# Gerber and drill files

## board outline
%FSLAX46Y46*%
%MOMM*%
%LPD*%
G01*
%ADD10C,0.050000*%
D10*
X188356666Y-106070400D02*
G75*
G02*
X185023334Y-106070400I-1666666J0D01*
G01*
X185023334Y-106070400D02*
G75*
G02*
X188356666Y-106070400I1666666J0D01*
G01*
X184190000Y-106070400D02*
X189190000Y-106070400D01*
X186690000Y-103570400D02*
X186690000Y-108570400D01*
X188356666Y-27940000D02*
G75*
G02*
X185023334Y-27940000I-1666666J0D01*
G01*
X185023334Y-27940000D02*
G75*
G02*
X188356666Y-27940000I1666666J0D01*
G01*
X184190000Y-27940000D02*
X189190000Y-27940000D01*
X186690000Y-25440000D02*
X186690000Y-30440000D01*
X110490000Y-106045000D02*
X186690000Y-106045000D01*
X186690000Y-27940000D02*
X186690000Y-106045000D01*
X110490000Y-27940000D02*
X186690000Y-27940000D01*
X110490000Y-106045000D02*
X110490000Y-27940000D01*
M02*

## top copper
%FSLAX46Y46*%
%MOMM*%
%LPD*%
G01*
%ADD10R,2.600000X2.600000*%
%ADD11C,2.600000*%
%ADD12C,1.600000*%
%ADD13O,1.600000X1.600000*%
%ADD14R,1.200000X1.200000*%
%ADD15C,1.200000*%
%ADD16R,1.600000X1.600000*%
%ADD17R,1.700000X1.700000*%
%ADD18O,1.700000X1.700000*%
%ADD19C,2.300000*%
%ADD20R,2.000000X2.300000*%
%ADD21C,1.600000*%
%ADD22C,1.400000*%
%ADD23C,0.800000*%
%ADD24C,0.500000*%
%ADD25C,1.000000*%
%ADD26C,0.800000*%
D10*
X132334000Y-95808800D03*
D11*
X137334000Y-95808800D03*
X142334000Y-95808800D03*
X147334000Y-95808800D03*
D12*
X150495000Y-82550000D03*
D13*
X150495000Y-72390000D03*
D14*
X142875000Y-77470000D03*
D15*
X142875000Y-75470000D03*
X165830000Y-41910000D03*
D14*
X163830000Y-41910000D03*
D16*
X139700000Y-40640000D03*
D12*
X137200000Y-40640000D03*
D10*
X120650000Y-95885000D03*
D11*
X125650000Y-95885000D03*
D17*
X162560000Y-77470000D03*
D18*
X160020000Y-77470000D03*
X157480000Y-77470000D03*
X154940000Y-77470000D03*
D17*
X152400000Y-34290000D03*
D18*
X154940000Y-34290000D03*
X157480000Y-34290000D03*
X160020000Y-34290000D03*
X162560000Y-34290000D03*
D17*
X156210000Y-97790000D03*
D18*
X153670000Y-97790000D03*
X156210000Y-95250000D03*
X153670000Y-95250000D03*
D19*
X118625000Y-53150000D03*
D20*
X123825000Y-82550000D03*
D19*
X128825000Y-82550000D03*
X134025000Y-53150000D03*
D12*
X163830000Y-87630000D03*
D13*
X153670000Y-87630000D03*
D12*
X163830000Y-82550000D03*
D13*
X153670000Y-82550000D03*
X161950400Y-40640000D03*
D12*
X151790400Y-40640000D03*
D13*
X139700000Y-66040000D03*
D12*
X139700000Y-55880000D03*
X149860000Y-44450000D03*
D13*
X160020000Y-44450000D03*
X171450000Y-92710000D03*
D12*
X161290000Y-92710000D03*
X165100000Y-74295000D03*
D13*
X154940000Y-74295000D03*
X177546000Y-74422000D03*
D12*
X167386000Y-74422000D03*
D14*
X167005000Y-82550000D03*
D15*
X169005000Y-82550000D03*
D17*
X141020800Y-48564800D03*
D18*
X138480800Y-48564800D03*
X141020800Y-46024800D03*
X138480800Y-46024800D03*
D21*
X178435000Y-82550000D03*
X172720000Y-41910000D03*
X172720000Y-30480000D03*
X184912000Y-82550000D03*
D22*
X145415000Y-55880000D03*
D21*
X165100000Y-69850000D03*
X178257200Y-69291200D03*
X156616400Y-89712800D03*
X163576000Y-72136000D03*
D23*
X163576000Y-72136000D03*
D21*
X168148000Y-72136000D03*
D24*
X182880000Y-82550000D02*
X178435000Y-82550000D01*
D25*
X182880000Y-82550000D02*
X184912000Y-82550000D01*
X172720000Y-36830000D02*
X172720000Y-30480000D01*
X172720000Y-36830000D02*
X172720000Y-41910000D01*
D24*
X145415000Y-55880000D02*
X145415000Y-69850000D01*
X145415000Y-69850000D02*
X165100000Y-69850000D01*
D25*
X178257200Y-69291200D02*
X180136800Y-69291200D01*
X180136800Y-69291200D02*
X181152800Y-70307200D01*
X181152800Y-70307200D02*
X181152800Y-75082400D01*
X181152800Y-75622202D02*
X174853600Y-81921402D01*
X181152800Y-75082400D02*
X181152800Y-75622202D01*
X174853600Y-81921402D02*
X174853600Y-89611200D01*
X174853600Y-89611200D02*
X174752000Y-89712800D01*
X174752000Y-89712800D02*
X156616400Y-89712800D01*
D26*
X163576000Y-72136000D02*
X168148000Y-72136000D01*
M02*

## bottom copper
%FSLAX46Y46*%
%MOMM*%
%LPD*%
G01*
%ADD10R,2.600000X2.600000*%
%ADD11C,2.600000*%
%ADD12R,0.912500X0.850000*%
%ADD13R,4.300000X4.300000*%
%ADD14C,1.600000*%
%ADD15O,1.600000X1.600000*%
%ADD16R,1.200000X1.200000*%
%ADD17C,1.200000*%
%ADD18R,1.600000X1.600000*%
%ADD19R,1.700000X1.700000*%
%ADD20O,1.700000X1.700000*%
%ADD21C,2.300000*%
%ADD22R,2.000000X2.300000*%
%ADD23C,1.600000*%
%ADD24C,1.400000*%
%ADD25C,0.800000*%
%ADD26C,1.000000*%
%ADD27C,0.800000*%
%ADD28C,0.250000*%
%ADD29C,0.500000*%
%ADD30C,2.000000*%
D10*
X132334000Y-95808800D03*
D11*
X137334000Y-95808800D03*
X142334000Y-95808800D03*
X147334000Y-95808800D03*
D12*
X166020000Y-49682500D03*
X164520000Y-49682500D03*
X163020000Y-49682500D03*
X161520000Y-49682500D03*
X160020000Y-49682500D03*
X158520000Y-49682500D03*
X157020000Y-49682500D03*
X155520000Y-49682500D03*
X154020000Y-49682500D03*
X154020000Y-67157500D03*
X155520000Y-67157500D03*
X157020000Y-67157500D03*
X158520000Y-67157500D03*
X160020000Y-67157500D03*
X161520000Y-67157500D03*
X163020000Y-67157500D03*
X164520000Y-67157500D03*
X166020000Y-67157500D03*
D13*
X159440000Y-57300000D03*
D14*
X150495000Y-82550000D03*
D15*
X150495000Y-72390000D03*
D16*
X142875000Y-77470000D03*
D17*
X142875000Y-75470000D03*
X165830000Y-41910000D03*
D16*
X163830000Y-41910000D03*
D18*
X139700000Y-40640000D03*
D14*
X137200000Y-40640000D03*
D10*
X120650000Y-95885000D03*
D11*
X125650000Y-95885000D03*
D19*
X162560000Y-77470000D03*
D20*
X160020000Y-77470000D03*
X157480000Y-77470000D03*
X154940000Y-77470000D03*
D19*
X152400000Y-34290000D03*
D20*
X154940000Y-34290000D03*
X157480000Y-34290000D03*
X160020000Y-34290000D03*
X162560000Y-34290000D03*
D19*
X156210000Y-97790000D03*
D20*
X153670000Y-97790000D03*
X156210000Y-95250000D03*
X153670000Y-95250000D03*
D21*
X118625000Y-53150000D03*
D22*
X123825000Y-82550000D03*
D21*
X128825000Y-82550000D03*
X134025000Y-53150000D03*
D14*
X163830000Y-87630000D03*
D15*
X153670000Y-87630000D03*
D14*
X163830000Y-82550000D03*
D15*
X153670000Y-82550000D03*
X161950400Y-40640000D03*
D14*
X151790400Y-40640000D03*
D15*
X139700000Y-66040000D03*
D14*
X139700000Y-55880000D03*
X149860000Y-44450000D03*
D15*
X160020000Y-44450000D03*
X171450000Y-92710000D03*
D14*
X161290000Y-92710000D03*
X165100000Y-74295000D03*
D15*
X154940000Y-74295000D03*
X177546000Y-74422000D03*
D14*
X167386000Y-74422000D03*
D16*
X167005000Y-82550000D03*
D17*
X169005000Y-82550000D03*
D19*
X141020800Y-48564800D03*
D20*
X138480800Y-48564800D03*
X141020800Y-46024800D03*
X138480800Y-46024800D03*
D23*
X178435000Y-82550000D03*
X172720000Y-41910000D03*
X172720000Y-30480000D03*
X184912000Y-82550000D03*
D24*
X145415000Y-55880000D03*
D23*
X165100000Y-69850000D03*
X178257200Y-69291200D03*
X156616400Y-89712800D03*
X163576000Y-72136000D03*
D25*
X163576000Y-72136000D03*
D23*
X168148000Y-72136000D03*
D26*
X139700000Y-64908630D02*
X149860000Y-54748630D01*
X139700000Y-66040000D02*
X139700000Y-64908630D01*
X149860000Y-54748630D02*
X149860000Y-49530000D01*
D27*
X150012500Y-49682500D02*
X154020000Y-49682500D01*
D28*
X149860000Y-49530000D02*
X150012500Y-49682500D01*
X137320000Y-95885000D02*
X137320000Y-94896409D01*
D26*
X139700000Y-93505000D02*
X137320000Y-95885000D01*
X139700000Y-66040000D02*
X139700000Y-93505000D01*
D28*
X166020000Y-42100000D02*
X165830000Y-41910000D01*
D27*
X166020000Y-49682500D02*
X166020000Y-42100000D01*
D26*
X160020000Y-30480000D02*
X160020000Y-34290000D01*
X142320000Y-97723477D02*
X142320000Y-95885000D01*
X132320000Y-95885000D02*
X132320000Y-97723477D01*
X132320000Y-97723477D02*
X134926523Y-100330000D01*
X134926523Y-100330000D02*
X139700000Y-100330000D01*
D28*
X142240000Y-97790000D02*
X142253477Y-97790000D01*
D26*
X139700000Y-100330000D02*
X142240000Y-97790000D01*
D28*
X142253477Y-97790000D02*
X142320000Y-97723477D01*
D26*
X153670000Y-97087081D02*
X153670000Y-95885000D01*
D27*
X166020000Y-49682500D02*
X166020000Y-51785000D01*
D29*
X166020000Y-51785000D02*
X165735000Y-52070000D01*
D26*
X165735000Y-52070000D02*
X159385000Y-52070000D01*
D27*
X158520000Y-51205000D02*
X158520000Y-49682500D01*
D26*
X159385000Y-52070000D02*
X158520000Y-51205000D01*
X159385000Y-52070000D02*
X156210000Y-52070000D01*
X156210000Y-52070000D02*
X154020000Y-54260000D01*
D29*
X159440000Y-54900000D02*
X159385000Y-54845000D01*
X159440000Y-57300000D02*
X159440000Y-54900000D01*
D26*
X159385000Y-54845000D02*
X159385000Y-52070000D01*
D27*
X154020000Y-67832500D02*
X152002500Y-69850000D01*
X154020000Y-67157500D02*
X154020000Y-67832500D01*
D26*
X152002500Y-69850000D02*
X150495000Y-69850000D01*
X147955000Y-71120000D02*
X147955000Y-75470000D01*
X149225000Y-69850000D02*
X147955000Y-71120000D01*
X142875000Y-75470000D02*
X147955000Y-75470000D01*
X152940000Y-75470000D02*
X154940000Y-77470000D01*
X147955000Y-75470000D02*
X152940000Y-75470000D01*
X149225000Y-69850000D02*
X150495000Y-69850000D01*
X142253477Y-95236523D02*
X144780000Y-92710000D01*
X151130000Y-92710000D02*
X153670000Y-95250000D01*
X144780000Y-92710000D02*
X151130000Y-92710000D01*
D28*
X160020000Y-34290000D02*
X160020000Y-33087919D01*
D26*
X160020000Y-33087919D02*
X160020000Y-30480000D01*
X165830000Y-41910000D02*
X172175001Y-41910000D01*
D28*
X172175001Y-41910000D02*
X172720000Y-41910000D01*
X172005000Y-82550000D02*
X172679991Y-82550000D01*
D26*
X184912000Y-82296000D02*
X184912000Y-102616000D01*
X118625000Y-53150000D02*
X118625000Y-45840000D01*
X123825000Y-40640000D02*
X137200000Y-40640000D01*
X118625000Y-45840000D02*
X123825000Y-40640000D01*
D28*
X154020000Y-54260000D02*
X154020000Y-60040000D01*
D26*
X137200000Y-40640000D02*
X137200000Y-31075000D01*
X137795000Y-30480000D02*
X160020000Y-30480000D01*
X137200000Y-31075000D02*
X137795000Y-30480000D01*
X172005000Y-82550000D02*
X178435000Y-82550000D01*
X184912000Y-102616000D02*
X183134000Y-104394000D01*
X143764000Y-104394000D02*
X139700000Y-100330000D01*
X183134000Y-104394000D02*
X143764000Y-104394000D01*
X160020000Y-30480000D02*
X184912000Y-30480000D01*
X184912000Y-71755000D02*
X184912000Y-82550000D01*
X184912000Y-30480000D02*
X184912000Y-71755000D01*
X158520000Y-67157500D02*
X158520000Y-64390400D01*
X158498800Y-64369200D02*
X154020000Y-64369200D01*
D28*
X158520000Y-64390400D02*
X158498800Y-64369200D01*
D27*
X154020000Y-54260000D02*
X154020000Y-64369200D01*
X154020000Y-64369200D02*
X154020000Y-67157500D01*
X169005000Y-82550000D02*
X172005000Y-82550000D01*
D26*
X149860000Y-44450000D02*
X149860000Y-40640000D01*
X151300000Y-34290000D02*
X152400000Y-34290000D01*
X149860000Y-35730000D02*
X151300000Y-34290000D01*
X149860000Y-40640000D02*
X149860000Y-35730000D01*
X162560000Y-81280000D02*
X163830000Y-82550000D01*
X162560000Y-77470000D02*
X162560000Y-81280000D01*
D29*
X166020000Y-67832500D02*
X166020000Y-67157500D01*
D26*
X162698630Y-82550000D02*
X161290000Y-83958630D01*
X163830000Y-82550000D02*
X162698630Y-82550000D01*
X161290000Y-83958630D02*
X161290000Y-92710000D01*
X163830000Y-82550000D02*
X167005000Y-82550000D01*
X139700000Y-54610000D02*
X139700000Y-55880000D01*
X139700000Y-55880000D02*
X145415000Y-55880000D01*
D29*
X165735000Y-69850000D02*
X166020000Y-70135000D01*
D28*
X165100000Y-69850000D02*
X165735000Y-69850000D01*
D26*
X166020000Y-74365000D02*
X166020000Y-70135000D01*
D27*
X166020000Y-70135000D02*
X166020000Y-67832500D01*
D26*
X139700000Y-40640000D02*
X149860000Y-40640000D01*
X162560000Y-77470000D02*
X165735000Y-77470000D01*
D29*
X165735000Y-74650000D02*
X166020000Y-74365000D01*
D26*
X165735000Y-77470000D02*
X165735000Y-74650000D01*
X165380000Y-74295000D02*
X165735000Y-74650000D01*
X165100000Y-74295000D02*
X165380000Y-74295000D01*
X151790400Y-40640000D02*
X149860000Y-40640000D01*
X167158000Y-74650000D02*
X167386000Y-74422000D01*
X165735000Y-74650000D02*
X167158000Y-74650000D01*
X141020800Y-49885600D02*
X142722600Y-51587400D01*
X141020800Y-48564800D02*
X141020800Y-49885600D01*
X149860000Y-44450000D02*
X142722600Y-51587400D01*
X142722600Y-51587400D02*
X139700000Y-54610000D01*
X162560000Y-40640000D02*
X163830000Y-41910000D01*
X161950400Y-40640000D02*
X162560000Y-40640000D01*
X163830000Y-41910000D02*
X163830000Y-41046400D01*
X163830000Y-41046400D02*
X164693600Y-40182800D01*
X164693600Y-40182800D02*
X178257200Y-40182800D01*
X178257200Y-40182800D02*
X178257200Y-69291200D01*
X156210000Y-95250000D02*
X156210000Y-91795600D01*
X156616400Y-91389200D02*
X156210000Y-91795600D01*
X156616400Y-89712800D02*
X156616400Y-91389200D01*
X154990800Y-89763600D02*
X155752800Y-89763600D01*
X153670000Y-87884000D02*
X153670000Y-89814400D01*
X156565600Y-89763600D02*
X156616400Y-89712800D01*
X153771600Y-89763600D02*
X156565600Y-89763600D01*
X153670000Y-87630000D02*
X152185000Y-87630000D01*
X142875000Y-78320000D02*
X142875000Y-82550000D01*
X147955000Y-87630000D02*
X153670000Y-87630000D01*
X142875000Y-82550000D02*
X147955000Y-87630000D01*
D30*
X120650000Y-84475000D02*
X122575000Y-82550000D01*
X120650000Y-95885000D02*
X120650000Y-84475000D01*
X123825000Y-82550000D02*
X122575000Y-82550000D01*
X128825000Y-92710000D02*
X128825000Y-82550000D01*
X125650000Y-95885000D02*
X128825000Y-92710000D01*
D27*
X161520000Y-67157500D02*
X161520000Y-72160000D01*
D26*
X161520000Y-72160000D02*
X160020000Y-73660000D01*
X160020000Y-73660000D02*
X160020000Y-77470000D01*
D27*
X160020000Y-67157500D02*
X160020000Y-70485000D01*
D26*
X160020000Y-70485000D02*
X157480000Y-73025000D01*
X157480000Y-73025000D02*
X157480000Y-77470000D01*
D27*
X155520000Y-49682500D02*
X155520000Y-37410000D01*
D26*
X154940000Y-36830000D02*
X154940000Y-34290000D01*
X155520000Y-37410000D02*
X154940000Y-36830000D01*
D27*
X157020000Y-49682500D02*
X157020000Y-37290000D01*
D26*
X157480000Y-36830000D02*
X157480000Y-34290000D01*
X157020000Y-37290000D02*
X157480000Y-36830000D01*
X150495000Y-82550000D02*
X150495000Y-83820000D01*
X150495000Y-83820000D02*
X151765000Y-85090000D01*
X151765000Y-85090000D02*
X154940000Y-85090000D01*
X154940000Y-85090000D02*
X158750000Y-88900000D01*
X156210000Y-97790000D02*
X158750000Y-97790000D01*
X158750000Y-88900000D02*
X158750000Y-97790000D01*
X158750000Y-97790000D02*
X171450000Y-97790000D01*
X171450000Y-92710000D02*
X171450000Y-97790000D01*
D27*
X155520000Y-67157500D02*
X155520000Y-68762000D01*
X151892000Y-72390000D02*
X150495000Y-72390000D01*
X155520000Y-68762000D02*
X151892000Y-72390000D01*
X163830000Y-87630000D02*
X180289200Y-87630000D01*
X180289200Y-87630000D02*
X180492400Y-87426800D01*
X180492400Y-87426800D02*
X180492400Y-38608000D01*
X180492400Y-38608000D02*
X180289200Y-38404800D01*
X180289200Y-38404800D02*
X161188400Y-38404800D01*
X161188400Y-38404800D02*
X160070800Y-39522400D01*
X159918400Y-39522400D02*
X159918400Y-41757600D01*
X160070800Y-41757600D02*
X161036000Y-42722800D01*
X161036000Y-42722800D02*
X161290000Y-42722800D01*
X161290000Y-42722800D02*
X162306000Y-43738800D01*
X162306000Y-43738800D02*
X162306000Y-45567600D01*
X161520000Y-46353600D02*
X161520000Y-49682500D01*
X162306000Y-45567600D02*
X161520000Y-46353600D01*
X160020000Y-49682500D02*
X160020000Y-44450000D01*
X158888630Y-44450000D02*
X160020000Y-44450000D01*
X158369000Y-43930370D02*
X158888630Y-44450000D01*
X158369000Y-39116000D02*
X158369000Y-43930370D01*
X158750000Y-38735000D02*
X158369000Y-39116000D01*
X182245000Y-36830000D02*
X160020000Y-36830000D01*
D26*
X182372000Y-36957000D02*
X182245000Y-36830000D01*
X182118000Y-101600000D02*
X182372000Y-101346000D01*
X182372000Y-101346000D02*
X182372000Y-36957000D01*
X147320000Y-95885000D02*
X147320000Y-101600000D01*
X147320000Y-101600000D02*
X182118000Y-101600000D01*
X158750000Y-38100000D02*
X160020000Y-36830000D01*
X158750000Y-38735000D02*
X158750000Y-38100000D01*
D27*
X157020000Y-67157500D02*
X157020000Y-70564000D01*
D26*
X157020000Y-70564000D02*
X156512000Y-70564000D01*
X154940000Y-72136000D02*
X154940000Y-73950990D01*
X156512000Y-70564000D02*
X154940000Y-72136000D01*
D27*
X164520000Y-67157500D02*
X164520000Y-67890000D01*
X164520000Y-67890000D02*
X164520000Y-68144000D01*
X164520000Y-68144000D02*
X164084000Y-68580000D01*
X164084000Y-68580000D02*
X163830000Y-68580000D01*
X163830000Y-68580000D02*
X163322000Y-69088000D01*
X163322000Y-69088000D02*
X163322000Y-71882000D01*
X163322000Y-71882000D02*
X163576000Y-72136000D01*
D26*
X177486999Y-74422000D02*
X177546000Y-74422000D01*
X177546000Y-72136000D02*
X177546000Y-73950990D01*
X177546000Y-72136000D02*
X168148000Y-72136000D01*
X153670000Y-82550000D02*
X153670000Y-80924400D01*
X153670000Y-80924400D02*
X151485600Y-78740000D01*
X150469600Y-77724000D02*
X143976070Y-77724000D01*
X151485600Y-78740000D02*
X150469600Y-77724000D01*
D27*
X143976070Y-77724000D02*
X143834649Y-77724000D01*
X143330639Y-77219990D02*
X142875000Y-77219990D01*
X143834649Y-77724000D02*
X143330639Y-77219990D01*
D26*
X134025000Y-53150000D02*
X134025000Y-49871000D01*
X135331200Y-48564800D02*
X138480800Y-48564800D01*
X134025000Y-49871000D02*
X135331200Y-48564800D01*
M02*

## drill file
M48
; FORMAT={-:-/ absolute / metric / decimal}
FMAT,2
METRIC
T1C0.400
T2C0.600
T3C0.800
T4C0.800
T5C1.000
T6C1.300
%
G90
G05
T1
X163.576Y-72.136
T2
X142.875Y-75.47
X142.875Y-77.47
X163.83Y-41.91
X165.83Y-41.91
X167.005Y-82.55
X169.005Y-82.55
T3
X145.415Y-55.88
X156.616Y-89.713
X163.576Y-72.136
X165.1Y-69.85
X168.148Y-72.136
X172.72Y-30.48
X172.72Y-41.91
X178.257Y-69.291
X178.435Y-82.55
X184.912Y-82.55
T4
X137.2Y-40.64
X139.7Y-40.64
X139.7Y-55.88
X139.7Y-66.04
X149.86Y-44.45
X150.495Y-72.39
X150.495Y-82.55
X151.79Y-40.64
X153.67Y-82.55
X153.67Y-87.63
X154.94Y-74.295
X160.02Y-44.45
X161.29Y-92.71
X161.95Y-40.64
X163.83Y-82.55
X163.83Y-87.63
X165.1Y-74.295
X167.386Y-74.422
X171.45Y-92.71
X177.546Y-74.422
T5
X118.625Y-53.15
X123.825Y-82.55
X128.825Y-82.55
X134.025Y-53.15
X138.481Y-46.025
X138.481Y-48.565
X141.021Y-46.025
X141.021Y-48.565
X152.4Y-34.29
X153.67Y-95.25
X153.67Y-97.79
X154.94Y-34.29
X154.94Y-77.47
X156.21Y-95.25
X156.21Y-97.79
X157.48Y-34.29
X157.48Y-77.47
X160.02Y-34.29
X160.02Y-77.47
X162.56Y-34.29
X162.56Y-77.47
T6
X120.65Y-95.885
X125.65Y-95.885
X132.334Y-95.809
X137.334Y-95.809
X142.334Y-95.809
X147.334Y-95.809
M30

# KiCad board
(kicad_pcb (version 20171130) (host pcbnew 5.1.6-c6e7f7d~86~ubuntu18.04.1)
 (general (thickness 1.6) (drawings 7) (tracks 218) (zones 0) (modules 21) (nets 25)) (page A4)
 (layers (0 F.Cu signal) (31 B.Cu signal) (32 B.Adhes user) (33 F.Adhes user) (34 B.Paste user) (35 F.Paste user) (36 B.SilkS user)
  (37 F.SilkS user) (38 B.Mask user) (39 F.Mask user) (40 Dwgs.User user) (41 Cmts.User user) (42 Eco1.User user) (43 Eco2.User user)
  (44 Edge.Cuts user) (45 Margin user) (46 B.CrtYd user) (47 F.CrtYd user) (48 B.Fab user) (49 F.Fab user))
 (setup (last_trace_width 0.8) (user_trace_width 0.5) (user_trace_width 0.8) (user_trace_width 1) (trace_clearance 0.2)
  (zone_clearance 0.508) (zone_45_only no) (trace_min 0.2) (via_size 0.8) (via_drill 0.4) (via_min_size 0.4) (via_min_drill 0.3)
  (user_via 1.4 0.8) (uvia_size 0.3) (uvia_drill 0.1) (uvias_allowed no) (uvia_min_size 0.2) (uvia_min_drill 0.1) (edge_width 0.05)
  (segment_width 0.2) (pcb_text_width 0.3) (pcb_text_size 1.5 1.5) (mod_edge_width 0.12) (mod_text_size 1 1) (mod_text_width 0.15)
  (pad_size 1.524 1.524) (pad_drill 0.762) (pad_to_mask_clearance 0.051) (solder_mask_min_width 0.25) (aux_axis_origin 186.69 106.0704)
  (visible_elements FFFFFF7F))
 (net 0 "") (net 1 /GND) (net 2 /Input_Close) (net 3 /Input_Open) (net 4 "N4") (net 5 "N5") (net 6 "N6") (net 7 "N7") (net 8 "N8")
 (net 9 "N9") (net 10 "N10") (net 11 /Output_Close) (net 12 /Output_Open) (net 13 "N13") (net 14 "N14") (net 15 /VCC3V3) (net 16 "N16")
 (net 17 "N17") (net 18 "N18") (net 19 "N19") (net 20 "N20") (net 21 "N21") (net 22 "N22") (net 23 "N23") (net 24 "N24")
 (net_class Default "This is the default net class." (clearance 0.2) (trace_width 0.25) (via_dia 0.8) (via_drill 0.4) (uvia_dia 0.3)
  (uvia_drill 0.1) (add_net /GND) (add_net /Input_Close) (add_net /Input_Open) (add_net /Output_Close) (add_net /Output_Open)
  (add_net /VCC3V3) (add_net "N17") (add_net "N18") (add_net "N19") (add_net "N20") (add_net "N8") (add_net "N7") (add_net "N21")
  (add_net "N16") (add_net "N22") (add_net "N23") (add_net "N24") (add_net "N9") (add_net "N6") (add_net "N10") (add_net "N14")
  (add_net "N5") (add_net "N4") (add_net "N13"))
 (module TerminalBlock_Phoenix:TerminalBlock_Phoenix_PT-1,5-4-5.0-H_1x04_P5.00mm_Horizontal (layer F.Cu) (at 132.334 95.8088)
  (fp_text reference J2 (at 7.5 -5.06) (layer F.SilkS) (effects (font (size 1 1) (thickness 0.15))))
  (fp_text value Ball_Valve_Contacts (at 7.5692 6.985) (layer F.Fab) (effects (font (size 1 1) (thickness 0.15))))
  (pad 4 thru_hole rect (at 0 0) (size 2.6 2.6) (drill 1.3) (layers *.Cu *.Mask) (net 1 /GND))
  (pad 3 thru_hole circle (at 5 0) (size 2.6 2.6) (drill 1.3) (layers *.Cu *.Mask) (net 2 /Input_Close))
  (pad 2 thru_hole circle (at 10 0) (size 2.6 2.6) (drill 1.3) (layers *.Cu *.Mask) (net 1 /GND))
  (pad 1 thru_hole circle (at 15 0) (size 2.6 2.6) (drill 1.3) (layers *.Cu *.Mask) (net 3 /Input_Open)))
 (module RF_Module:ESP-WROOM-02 (layer B.Cu) (at 160.02 58.42 90)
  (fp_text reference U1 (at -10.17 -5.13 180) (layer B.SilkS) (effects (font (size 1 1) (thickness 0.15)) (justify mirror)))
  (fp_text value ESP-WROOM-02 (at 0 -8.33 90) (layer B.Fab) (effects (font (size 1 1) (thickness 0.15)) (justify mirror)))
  (pad 18 smd rect (at 8.7375 6 90) (size 0.85 0.9125) (layers B.Cu B.Paste B.Mask) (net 1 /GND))
  (pad 17 smd rect (at 8.7375 4.5 90) (size 0.85 0.9125) (layers B.Cu B.Paste B.Mask) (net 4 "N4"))
  (pad 16 smd rect (at 8.7375 3 90) (size 0.85 0.9125) (layers B.Cu B.Paste B.Mask) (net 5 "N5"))
  (pad 15 smd rect (at 8.7375 1.5 90) (size 0.85 0.9125) (layers B.Cu B.Paste B.Mask) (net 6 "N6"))
  (pad 14 smd rect (at 8.7375 0 90) (size 0.85 0.9125) (layers B.Cu B.Paste B.Mask) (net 3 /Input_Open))
  (pad 13 smd rect (at 8.7375 -1.5 90) (size 0.85 0.9125) (layers B.Cu B.Paste B.Mask) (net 1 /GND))
  (pad 12 smd rect (at 8.7375 -3 90) (size 0.85 0.9125) (layers B.Cu B.Paste B.Mask) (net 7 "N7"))
  (pad 11 smd rect (at 8.7375 -4.5 90) (size 0.85 0.9125) (layers B.Cu B.Paste B.Mask) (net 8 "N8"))
  (pad 10 smd rect (at 8.7375 -6 90) (size 0.85 0.9125) (layers B.Cu B.Paste B.Mask) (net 2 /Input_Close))
  (pad 9 smd rect (at -8.7375 -6 90) (size 0.85 0.9125) (layers B.Cu B.Paste B.Mask) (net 1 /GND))
  (pad 8 smd rect (at -8.7375 -4.5 90) (size 0.85 0.9125) (layers B.Cu B.Paste B.Mask) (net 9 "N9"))
  (pad 7 smd rect (at -8.7375 -3 90) (size 0.85 0.9125) (layers B.Cu B.Paste B.Mask) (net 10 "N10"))
  (pad 6 smd rect (at -8.7375 -1.5 90) (size 0.85 0.9125) (layers B.Cu B.Paste B.Mask) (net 1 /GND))
  (pad 5 smd rect (at -8.7375 0 90) (size 0.85 0.9125) (layers B.Cu B.Paste B.Mask) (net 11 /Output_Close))
  (pad 4 smd rect (at -8.7375 1.5 90) (size 0.85 0.9125) (layers B.Cu B.Paste B.Mask) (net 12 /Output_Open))
  (pad 3 smd rect (at -8.7375 3 90) (size 0.85 0.9125) (layers B.Cu B.Paste B.Mask) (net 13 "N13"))
  (pad 2 smd rect (at -8.7375 4.5 90) (size 0.85 0.9125) (layers B.Cu B.Paste B.Mask) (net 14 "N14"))
  (pad 1 smd rect (at -8.7375 6 90) (size 0.85 0.9125) (layers B.Cu B.Paste B.Mask) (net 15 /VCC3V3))
  (pad 19 smd rect (at 1.12 -0.58 90) (size 4.3 4.3) (layers B.Cu B.Paste B.Mask) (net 1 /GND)))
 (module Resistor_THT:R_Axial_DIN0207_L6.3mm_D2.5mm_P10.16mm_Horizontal (layer F.Cu) (at 150.495 82.55 90)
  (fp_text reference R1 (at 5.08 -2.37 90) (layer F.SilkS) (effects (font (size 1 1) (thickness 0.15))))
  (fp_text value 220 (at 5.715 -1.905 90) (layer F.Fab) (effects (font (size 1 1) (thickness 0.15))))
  (pad 1 thru_hole circle (at 0 0 90) (size 1.6 1.6) (drill 0.8) (layers *.Cu *.Mask) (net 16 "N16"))
  (pad 2 thru_hole oval (at 10.16 0 90) (size 1.6 1.6) (drill 0.8) (layers *.Cu *.Mask) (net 9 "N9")))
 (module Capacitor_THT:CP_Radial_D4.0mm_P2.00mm (layer F.Cu) (at 142.875 77.47 90)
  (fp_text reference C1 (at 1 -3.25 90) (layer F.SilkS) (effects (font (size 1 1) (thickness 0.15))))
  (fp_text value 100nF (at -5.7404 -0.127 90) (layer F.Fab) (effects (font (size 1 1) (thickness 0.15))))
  (pad 1 thru_hole rect (at 0 0 90) (size 1.2 1.2) (drill 0.6) (layers *.Cu *.Mask) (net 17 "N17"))
  (pad 2 thru_hole circle (at 2 0 90) (size 1.2 1.2) (drill 0.6) (layers *.Cu *.Mask) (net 1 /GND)))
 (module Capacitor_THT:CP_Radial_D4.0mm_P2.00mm (layer F.Cu) (at 163.83 41.91)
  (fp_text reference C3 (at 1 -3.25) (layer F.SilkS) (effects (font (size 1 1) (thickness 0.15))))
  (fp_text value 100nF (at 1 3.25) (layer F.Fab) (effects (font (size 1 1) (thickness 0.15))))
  (pad 2 thru_hole circle (at 2 0) (size 1.2 1.2) (drill 0.6) (layers *.Cu *.Mask) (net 1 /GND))
  (pad 1 thru_hole rect (at 0 0) (size 1.2 1.2) (drill 0.6) (layers *.Cu *.Mask) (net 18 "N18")))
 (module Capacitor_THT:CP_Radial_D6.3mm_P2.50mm (layer F.Cu) (at 139.7 40.64 180)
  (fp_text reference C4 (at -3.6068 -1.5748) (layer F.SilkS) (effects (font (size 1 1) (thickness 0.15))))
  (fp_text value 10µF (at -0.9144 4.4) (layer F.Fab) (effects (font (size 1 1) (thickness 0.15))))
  (pad 1 thru_hole rect (at 0 0 180) (size 1.6 1.6) (drill 0.8) (layers *.Cu *.Mask) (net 15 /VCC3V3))
  (pad 2 thru_hole circle (at 2.5 0 180) (size 1.6 1.6) (drill 0.8) (layers *.Cu *.Mask) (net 1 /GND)))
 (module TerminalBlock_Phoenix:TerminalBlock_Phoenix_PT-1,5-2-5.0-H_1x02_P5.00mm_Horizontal (layer F.Cu) (at 120.65 95.885)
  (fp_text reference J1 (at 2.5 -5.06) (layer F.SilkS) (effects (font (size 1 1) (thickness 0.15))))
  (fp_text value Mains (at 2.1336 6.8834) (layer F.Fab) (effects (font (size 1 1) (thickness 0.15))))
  (pad 1 thru_hole rect (at 0 0) (size 2.6 2.6) (drill 1.3) (layers *.Cu *.Mask) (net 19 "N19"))
  (pad 2 thru_hole circle (at 5 0) (size 2.6 2.6) (drill 1.3) (layers *.Cu *.Mask) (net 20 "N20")))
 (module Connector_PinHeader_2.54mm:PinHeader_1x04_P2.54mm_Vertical (layer F.Cu) (at 162.56 77.47 270)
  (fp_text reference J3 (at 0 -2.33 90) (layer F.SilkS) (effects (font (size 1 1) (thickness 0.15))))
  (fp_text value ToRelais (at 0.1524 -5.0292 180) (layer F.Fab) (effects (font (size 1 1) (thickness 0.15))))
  (pad 1 thru_hole rect (at 0 0 270) (size 1.7 1.7) (drill 1) (layers *.Cu *.Mask) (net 15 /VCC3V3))
  (pad 2 thru_hole oval (at 0 2.54 270) (size 1.7 1.7) (drill 1) (layers *.Cu *.Mask) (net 12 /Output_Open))
  (pad 3 thru_hole oval (at 0 5.08 270) (size 1.7 1.7) (drill 1) (layers *.Cu *.Mask) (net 11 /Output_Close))
  (pad 4 thru_hole oval (at 0 7.62 270) (size 1.7 1.7) (drill 1) (layers *.Cu *.Mask) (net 1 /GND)))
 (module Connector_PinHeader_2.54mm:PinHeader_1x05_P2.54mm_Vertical (layer F.Cu) (at 152.4 34.29 90)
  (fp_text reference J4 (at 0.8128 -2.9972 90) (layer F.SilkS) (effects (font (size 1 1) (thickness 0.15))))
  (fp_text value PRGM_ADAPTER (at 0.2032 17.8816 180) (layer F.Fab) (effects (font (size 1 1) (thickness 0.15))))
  (pad 1 thru_hole rect (at 0 0 90) (size 1.7 1.7) (drill 1) (layers *.Cu *.Mask) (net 15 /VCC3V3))
  (pad 2 thru_hole oval (at 0 2.54 90) (size 1.7 1.7) (drill 1) (layers *.Cu *.Mask) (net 8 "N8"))
  (pad 3 thru_hole oval (at 0 5.08 90) (size 1.7 1.7) (drill 1) (layers *.Cu *.Mask) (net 7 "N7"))
  (pad 4 thru_hole oval (at 0 7.62 90) (size 1.7 1.7) (drill 1) (layers *.Cu *.Mask) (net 1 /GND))
  (pad 5 thru_hole oval (at 0 10.16 90) (size 1.7 1.7) (drill 1) (layers *.Cu *.Mask) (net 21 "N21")))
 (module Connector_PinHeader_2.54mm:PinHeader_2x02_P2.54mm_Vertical (layer F.Cu) (at 156.21 97.79 180)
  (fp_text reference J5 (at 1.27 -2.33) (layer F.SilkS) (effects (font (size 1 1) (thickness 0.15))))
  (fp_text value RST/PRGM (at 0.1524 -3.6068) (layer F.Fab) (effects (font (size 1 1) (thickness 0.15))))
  (pad 1 thru_hole rect (at 0 0 180) (size 1.7 1.7) (drill 1) (layers *.Cu *.Mask) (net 16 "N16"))
  (pad 2 thru_hole oval (at 2.54 0 180) (size 1.7 1.7) (drill 1) (layers *.Cu *.Mask) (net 1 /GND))
  (pad 3 thru_hole oval (at 0 2.54 180) (size 1.7 1.7) (drill 1) (layers *.Cu *.Mask) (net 18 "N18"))
  (pad 4 thru_hole oval (at 2.54 2.54 180) (size 1.7 1.7) (drill 1) (layers *.Cu *.Mask) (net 1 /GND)))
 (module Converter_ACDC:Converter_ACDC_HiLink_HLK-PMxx (layer F.Cu) (at 123.825 82.55 90)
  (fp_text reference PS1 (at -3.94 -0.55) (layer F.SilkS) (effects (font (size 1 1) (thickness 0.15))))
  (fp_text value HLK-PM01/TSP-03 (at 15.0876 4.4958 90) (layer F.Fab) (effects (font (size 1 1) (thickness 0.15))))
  (pad 3 thru_hole circle (at 29.4 -5.2 90) (size 2.3 2.3) (drill 1) (layers *.Cu *.Mask) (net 1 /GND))
  (pad 1 thru_hole rect (at 0 0 90) (size 2.3 2) (drill 1) (layers *.Cu *.Mask) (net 19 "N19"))
  (pad 2 thru_hole circle (at 0 5 90) (size 2.3 2.3) (drill 1) (layers *.Cu *.Mask) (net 20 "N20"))
  (pad 4 thru_hole circle (at 29.4 10.2 90) (size 2.3 2.3) (drill 1) (layers *.Cu *.Mask) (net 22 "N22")))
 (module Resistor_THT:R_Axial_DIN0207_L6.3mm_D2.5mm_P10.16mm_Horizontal (layer F.Cu) (at 163.83 87.63 180)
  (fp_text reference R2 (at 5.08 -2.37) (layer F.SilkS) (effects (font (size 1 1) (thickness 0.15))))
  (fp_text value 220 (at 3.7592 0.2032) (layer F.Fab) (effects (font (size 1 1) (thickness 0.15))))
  (pad 1 thru_hole circle (at 0 0 180) (size 1.6 1.6) (drill 0.8) (layers *.Cu *.Mask) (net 6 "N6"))
  (pad 2 thru_hole oval (at 10.16 0 180) (size 1.6 1.6) (drill 0.8) (layers *.Cu *.Mask) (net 18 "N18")))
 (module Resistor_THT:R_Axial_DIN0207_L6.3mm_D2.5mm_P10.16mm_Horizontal (layer F.Cu) (at 163.83 82.55 180)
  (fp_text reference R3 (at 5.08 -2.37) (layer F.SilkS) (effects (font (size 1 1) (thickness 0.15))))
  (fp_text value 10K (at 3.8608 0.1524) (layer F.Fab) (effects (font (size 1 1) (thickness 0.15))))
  (pad 1 thru_hole circle (at 0 0 180) (size 1.6 1.6) (drill 0.8) (layers *.Cu *.Mask) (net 15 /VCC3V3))
  (pad 2 thru_hole oval (at 10.16 0 180) (size 1.6 1.6) (drill 0.8) (layers *.Cu *.Mask) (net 17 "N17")))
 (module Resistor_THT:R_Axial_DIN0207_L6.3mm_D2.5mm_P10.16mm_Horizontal (layer F.Cu) (at 151.7904 40.64)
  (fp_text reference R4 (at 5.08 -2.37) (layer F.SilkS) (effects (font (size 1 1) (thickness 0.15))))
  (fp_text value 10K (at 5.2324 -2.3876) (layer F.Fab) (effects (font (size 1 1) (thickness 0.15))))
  (pad 2 thru_hole oval (at 10.16 0) (size 1.6 1.6) (drill 0.8) (layers *.Cu *.Mask) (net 18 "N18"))
  (pad 1 thru_hole circle (at 0 0) (size 1.6 1.6) (drill 0.8) (layers *.Cu *.Mask) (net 15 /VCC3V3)))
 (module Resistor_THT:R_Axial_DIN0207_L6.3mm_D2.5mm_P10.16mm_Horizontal (layer F.Cu) (at 139.7 55.88 270)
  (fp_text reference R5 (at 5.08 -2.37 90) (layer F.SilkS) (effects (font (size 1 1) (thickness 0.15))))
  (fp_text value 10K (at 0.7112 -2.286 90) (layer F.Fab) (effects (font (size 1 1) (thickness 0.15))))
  (pad 2 thru_hole oval (at 10.16 0 270) (size 1.6 1.6) (drill 0.8) (layers *.Cu *.Mask) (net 2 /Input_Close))
  (pad 1 thru_hole circle (at 0 0 270) (size 1.6 1.6) (drill 0.8) (layers *.Cu *.Mask) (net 15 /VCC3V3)))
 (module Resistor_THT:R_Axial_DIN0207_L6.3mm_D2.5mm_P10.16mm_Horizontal (layer F.Cu) (at 149.86 44.45)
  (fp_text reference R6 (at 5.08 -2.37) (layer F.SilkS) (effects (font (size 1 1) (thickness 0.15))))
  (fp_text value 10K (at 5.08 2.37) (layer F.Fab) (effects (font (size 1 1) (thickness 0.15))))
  (pad 1 thru_hole circle (at 0 0) (size 1.6 1.6) (drill 0.8) (layers *.Cu *.Mask) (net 15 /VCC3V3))
  (pad 2 thru_hole oval (at 10.16 0) (size 1.6 1.6) (drill 0.8) (layers *.Cu *.Mask) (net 3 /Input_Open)))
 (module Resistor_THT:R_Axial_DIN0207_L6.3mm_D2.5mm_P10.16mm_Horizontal (layer F.Cu) (at 161.29 92.71)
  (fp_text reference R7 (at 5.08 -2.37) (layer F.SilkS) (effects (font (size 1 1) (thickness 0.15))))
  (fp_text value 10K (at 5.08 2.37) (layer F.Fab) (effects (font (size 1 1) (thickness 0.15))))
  (pad 2 thru_hole oval (at 10.16 0) (size 1.6 1.6) (drill 0.8) (layers *.Cu *.Mask) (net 16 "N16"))
  (pad 1 thru_hole circle (at 0 0) (size 1.6 1.6) (drill 0.8) (layers *.Cu *.Mask) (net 15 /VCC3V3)))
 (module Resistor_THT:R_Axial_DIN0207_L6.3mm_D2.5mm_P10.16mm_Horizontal (layer F.Cu) (at 165.1 74.295 180)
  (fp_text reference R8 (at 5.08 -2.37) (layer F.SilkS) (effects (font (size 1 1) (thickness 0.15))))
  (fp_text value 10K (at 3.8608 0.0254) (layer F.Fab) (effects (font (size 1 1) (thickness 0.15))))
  (pad 1 thru_hole circle (at 0 0 180) (size 1.6 1.6) (drill 0.8) (layers *.Cu *.Mask) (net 15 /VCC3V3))
  (pad 2 thru_hole oval (at 10.16 0 180) (size 1.6 1.6) (drill 0.8) (layers *.Cu *.Mask) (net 10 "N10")))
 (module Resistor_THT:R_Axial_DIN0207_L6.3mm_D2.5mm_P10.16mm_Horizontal (layer F.Cu) (at 167.386 74.422)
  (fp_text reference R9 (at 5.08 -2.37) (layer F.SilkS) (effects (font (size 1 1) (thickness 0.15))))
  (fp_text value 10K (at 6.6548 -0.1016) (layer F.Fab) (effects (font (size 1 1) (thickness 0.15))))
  (pad 2 thru_hole oval (at 10.16 0) (size 1.6 1.6) (drill 0.8) (layers *.Cu *.Mask) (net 14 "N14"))
  (pad 1 thru_hole circle (at 0 0) (size 1.6 1.6) (drill 0.8) (layers *.Cu *.Mask) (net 15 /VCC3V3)))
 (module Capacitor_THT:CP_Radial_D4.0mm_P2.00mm (layer F.Cu) (at 167.005 82.55)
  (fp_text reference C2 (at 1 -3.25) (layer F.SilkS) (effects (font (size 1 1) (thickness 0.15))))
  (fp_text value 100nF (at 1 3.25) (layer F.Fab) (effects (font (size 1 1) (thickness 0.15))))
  (pad 1 thru_hole rect (at 0 0) (size 1.2 1.2) (drill 0.6) (layers *.Cu *.Mask) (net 15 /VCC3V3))
  (pad 2 thru_hole circle (at 2 0) (size 1.2 1.2) (drill 0.6) (layers *.Cu *.Mask) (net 1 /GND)))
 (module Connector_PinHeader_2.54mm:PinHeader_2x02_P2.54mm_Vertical (layer F.Cu) (at 141.0208 48.5648 180)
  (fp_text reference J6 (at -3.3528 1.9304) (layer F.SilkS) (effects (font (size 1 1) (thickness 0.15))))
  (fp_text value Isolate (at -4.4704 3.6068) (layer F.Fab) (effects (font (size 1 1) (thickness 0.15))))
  (pad 1 thru_hole rect (at 0 0 180) (size 1.7 1.7) (drill 1) (layers *.Cu *.Mask) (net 15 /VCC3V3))
  (pad 2 thru_hole oval (at 2.54 0 180) (size 1.7 1.7) (drill 1) (layers *.Cu *.Mask) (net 22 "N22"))
  (pad 3 thru_hole oval (at 0 2.54 180) (size 1.7 1.7) (drill 1) (layers *.Cu *.Mask) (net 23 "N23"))
  (pad 4 thru_hole oval (at 2.54 2.54 180) (size 1.7 1.7) (drill 1) (layers *.Cu *.Mask) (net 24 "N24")))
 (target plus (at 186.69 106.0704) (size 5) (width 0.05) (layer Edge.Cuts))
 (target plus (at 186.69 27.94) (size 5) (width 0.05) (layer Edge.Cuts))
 (gr_line (start 110.49 106.045) (end 186.69 106.045) (layer Edge.Cuts) (width 0.05))
 (gr_line (start 186.69 27.94) (end 186.69 106.045) (layer Edge.Cuts) (width 0.05))
 (gr_line (start 110.49 27.94) (end 186.69 27.94) (layer Edge.Cuts) (width 0.05))
 (gr_line (start 110.49 106.045) (end 110.49 27.94) (layer Edge.Cuts) (width 0.05))
 (segment (start 139.7 64.90863) (end 149.86 54.74863) (width 1) (layer B.Cu) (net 2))
 (segment (start 139.7 66.04) (end 139.7 64.90863) (width 1) (layer B.Cu) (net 2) (status 10))
 (segment (start 149.86 54.74863) (end 149.86 49.53) (width 1) (layer B.Cu) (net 2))
 (segment (start 150.0125 49.6825) (end 154.02 49.6825) (width 0.8) (layer B.Cu) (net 2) (status 20))
 (segment (start 149.86 49.53) (end 150.0125 49.6825) (width 0.25) (layer B.Cu) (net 2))
 (segment (start 137.32 95.885) (end 137.32 94.896409) (width 0.25) (layer B.Cu) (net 2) (status 30))
 (segment (start 139.7 93.505) (end 137.32 95.885) (width 1) (layer B.Cu) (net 2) (status 20))
 (segment (start 139.7 66.04) (end 139.7 93.505) (width 1) (layer B.Cu) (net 2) (status 10))
 (via (at 178.435 82.55) (size 1.6) (drill 0.8) (layers F.Cu B.Cu) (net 1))
 (via (at 172.72 41.91) (size 1.6) (drill 0.8) (layers F.Cu B.Cu) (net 1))
 (segment (start 166.02 42.1) (end 165.83 41.91) (width 0.25) (layer B.Cu) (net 1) (status 30))
 (segment (start 166.02 49.6825) (end 166.02 42.1) (width 0.8) (layer B.Cu) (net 1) (status 30))
 (segment (start 160.02 30.48) (end 160.02 34.29) (width 1) (layer B.Cu) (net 1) (status 20))
 (segment (start 142.32 97.723477) (end 142.32 95.885) (width 1) (layer B.Cu) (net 1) (status 20))
 (segment (start 132.32 95.885) (end 132.32 97.723477) (width 1) (layer B.Cu) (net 1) (status 10))
 (segment (start 132.32 97.723477) (end 134.926523 100.33) (width 1) (layer B.Cu) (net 1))
 (segment (start 134.926523 100.33) (end 139.7 100.33) (width 1) (layer B.Cu) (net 1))
 (segment (start 142.24 97.79) (end 142.253477 97.79) (width 0.25) (layer B.Cu) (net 1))
 (segment (start 139.7 100.33) (end 142.24 97.79) (width 1) (layer B.Cu) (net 1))
 (segment (start 142.253477 97.79) (end 142.32 97.723477) (width 0.25) (layer B.Cu) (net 1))
 (segment (start 153.67 97.087081) (end 153.67 95.885) (width 1) (layer B.Cu) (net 1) (status 30))
 (segment (start 166.02 49.6825) (end 166.02 51.785) (width 0.8) (layer B.Cu) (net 1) (status 10))
 (segment (start 166.02 51.785) (end 165.735 52.07) (width 0.5) (layer B.Cu) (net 1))
 (segment (start 165.735 52.07) (end 159.385 52.07) (width 1) (layer B.Cu) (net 1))
 (segment (start 158.52 51.205) (end 158.52 49.6825) (width 0.8) (layer B.Cu) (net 1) (status 20))
 (segment (start 159.385 52.07) (end 158.52 51.205) (width 1) (layer B.Cu) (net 1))
 (segment (start 159.385 52.07) (end 156.21 52.07) (width 1) (layer B.Cu) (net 1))
 (segment (start 156.21 52.07) (end 154.02 54.26) (width 1) (layer B.Cu) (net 1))
 (segment (start 159.44 54.9) (end 159.385 54.845) (width 0.5) (layer B.Cu) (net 1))
 (segment (start 159.44 57.3) (end 159.44 54.9) (width 0.5) (layer B.Cu) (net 1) (status 10))
 (segment (start 159.385 54.845) (end 159.385 52.07) (width 1) (layer B.Cu) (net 1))
 (segment (start 154.02 67.8325) (end 152.0025 69.85) (width 0.8) (layer B.Cu) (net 1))
 (segment (start 154.02 67.1575) (end 154.02 67.8325) (width 0.8) (layer B.Cu) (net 1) (status 10))
 (segment (start 152.0025 69.85) (end 150.495 69.85) (width 1) (layer B.Cu) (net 1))
 (segment (start 147.955 71.12) (end 147.955 75.47) (width 1) (layer B.Cu) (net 1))
 (segment (start 149.225 69.85) (end 147.955 71.12) (width 1) (layer B.Cu) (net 1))
 (segment (start 142.875 75.47) (end 147.955 75.47) (width 1) (layer B.Cu) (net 1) (status 10))
 (segment (start 152.94 75.47) (end 154.94 77.47) (width 1) (layer B.Cu) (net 1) (status 20))
 (segment (start 147.955 75.47) (end 152.94 75.47) (width 1) (layer B.Cu) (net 1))
 (segment (start 149.225 69.85) (end 150.495 69.85) (width 1) (layer B.Cu) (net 1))
 (segment (start 142.253477 95.236523) (end 144.78 92.71) (width 1) (layer B.Cu) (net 1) (status 10))
 (segment (start 151.13 92.71) (end 153.67 95.25) (width 1) (layer B.Cu) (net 1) (status 20))
 (segment (start 144.78 92.71) (end 151.13 92.71) (width 1) (layer B.Cu) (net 1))
 (segment (start 160.02 34.29) (end 160.02 33.087919) (width 0.25) (layer B.Cu) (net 1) (status 10))
 (segment (start 160.02 33.087919) (end 160.02 30.48) (width 1) (layer B.Cu) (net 1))
 (via (at 172.72 30.48) (size 1.6) (drill 0.8) (layers F.Cu B.Cu) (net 1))
 (segment (start 165.83 41.91) (end 172.175001 41.91) (width 1) (layer B.Cu) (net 1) (status 10))
 (segment (start 172.175001 41.91) (end 172.72 41.91) (width 0.25) (layer B.Cu) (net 1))
 (via (at 184.912 82.55) (size 1.6) (drill 0.8) (layers F.Cu B.Cu) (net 1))
 (segment (start 172.005 82.55) (end 172.679991 82.55) (width 0.25) (layer B.Cu) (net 1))
 (segment (start 184.912 82.296) (end 184.912 102.616) (width 1) (layer B.Cu) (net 1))
 (segment (start 182.88 82.55) (end 178.435 82.55) (width 0.5) (layer F.Cu) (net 1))
 (segment (start 118.625 53.15) (end 118.625 45.84) (width 1) (layer B.Cu) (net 1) (status 10))
 (segment (start 123.825 40.64) (end 137.2 40.64) (width 1) (layer B.Cu) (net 1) (status 20))
 (segment (start 118.625 45.84) (end 123.825 40.64) (width 1) (layer B.Cu) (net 1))
 (segment (start 154.02 54.26) (end 154.02 60.04) (width 0.25) (layer B.Cu) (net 1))
 (segment (start 137.2 40.64) (end 137.2 31.075) (width 1) (layer B.Cu) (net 1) (status 10))
 (segment (start 137.795 30.48) (end 160.02 30.48) (width 1) (layer B.Cu) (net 1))
 (segment (start 137.2 31.075) (end 137.795 30.48) (width 1) (layer B.Cu) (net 1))
 (segment (start 172.005 82.55) (end 178.435 82.55) (width 1) (layer B.Cu) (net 1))
 (segment (start 182.88 82.55) (end 184.912 82.55) (width 1) (layer F.Cu) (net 1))
 (segment (start 184.912 102.616) (end 183.134 104.394) (width 1) (layer B.Cu) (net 1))
 (segment (start 143.764 104.394) (end 139.7 100.33) (width 1) (layer B.Cu) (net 1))
 (segment (start 183.134 104.394) (end 143.764 104.394) (width 1) (layer B.Cu) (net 1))
 (segment (start 172.72 36.83) (end 172.72 30.48) (width 1) (layer F.Cu) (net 1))
 (segment (start 172.72 36.83) (end 172.72 41.91) (width 1) (layer F.Cu) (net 1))
 (segment (start 160.02 30.48) (end 184.912 30.48) (width 1) (layer B.Cu) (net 1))
 (segment (start 184.912 71.755) (end 184.912 82.55) (width 1) (layer B.Cu) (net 1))
 (segment (start 184.912 30.48) (end 184.912 71.755) (width 1) (layer B.Cu) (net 1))
 (segment (start 158.52 67.1575) (end 158.52 64.3904) (width 1) (layer B.Cu) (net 1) (status 10))
 (segment (start 158.4988 64.3692) (end 154.02 64.3692) (width 1) (layer B.Cu) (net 1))
 (segment (start 158.52 64.3904) (end 158.4988 64.3692) (width 0.25) (layer B.Cu) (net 1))
 (segment (start 154.02 54.26) (end 154.02 64.3692) (width 0.8) (layer B.Cu) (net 1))
 (segment (start 154.02 64.3692) (end 154.02 67.1575) (width 0.8) (layer B.Cu) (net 1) (status 20))
 (segment (start 169.005 82.55) (end 172.005 82.55) (width 0.8) (layer B.Cu) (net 1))
 (segment (start 149.86 44.45) (end 149.86 40.64) (width 1) (layer B.Cu) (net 15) (status 10))
 (segment (start 151.3 34.29) (end 152.4 34.29) (width 1) (layer B.Cu) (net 15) (status 20))
 (segment (start 149.86 35.73) (end 151.3 34.29) (width 1) (layer B.Cu) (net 15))
 (segment (start 149.86 40.64) (end 149.86 35.73) (width 1) (layer B.Cu) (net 15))
 (segment (start 162.56 81.28) (end 163.83 82.55) (width 1) (layer B.Cu) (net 15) (status 20))
 (segment (start 162.56 77.47) (end 162.56 81.28) (width 1) (layer B.Cu) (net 15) (status 10))
 (segment (start 166.02 67.8325) (end 166.02 67.1575) (width 0.5) (layer B.Cu) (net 15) (status 20))
 (segment (start 162.69863 82.55) (end 161.29 83.95863) (width 1) (layer B.Cu) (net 15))
 (segment (start 163.83 82.55) (end 162.69863 82.55) (width 1) (layer B.Cu) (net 15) (status 10))
 (segment (start 161.29 83.95863) (end 161.29 92.71) (width 1) (layer B.Cu) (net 15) (status 20))
 (segment (start 163.83 82.55) (end 167.005 82.55) (width 1) (layer B.Cu) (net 15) (status 30))
 (segment (start 139.7 54.61) (end 139.7 55.88) (width 1) (layer B.Cu) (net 15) (status 20))
 (segment (start 139.7 55.88) (end 145.415 55.88) (width 1) (layer B.Cu) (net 15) (status 10))
 (via (at 145.415 55.88) (size 1.4) (drill 0.8) (layers F.Cu B.Cu) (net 15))
 (segment (start 145.415 55.88) (end 145.415 69.85) (width 0.5) (layer F.Cu) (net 15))
 (segment (start 145.415 69.85) (end 165.1 69.85) (width 0.5) (layer F.Cu) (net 15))
 (via (at 165.1 69.85) (size 1.6) (drill 0.8) (layers F.Cu B.Cu) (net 15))
 (segment (start 165.735 69.85) (end 166.02 70.135) (width 0.5) (layer B.Cu) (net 15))
 (segment (start 165.1 69.85) (end 165.735 69.85) (width 0.25) (layer B.Cu) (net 15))
 (segment (start 166.02 74.365) (end 166.02 70.135) (width 1) (layer B.Cu) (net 15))
 (segment (start 166.02 70.135) (end 166.02 67.8325) (width 0.8) (layer B.Cu) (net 15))
 (segment (start 139.7 40.64) (end 149.86 40.64) (width 1) (layer B.Cu) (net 15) (status 10))
 (segment (start 162.56 77.47) (end 165.735 77.47) (width 1) (layer B.Cu) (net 15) (status 10))
 (segment (start 165.735 74.65) (end 166.02 74.365) (width 0.5) (layer B.Cu) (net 15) (status 10))
 (segment (start 165.735 77.47) (end 165.735 74.65) (width 1) (layer B.Cu) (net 15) (status 20))
 (segment (start 165.38 74.295) (end 165.735 74.65) (width 1) (layer B.Cu) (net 15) (status 30))
 (segment (start 165.1 74.295) (end 165.38 74.295) (width 1) (layer B.Cu) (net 15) (status 30))
 (segment (start 151.7904 40.64) (end 149.86 40.64) (width 1) (layer B.Cu) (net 15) (status 10))
 (segment (start 167.158 74.65) (end 167.386 74.422) (width 1) (layer B.Cu) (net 15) (status 30))
 (segment (start 165.735 74.65) (end 167.158 74.65) (width 1) (layer B.Cu) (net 15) (status 30))
 (segment (start 141.0208 49.8856) (end 142.7226 51.5874) (width 1) (layer B.Cu) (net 15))
 (segment (start 141.0208 48.5648) (end 141.0208 49.8856) (width 1) (layer B.Cu) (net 15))
 (segment (start 149.86 44.45) (end 142.7226 51.5874) (width 1) (layer B.Cu) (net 15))
 (segment (start 142.7226 51.5874) (end 139.7 54.61) (width 1) (layer B.Cu) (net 15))
 (segment (start 162.56 40.64) (end 163.83 41.91) (width 1) (layer B.Cu) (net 18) (status 30))
 (segment (start 161.9504 40.64) (end 162.56 40.64) (width 1) (layer B.Cu) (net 18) (status 30))
 (segment (start 163.83 41.91) (end 163.83 41.0464) (width 1) (layer B.Cu) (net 18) (status 10))
 (segment (start 163.83 41.0464) (end 164.6936 40.1828) (width 1) (layer B.Cu) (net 18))
 (segment (start 164.6936 40.1828) (end 178.2572 40.1828) (width 1) (layer B.Cu) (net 18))
 (segment (start 178.2572 40.1828) (end 178.2572 69.2912) (width 1) (layer B.Cu) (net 18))
 (segment (start 156.21 95.25) (end 156.21 91.7956) (width 1) (layer B.Cu) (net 18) (status 10))
 (via (at 178.2572 69.2912) (size 1.6) (drill 0.8) (layers F.Cu B.Cu) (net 18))
 (segment (start 178.2572 69.2912) (end 180.1368 69.2912) (width 1) (layer F.Cu) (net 18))
 (segment (start 180.1368 69.2912) (end 181.1528 70.3072) (width 1) (layer F.Cu) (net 18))
 (segment (start 181.1528 70.3072) (end 181.1528 75.0824) (width 1) (layer F.Cu) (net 18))
 (segment (start 181.1528 75.622202) (end 174.8536 81.921402) (width 1) (layer F.Cu) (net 18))
 (segment (start 181.1528 75.0824) (end 181.1528 75.622202) (width 1) (layer F.Cu) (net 18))
 (segment (start 174.8536 81.921402) (end 174.8536 89.6112) (width 1) (layer F.Cu) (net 18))
 (segment (start 174.8536 89.6112) (end 174.752 89.7128) (width 1) (layer F.Cu) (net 18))
 (segment (start 174.752 89.7128) (end 156.6164 89.7128) (width 1) (layer F.Cu) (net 18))
 (via (at 156.6164 89.7128) (size 1.6) (drill 0.8) (layers F.Cu B.Cu) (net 18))
 (segment (start 156.6164 91.3892) (end 156.21 91.7956) (width 1) (layer B.Cu) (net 18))
 (segment (start 156.6164 89.7128) (end 156.6164 91.3892) (width 1) (layer B.Cu) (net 18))
 (segment (start 154.9908 89.7636) (end 155.7528 89.7636) (width 1) (layer B.Cu) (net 18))
 (segment (start 153.67 87.884) (end 153.67 89.8144) (width 1) (layer B.Cu) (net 18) (status 10))
 (segment (start 156.5656 89.7636) (end 156.6164 89.7128) (width 1) (layer B.Cu) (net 18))
 (segment (start 153.7716 89.7636) (end 156.5656 89.7636) (width 1) (layer B.Cu) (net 18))
 (segment (start 153.67 87.63) (end 152.185 87.63) (width 1) (layer B.Cu) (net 18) (status 10))
 (segment (start 142.875 78.32) (end 142.875 82.55) (width 1) (layer B.Cu) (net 18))
 (segment (start 147.955 87.63) (end 153.67 87.63) (width 1) (layer B.Cu) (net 18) (status 20))
 (segment (start 142.875 82.55) (end 147.955 87.63) (width 1) (layer B.Cu) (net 18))
 (segment (start 120.65 84.475) (end 122.575 82.55) (width 2) (layer B.Cu) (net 19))
 (segment (start 120.65 95.885) (end 120.65 84.475) (width 2) (layer B.Cu) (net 19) (status 10))
 (segment (start 123.825 82.55) (end 122.575 82.55) (width 2) (layer B.Cu) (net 19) (status 10))
 (segment (start 128.825 92.71) (end 128.825 82.55) (width 2) (layer B.Cu) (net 20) (status 20))
 (segment (start 125.65 95.885) (end 128.825 92.71) (width 2) (layer B.Cu) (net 20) (status 10))
 (segment (start 161.52 67.1575) (end 161.52 72.16) (width 0.8) (layer B.Cu) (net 12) (status 10))
 (segment (start 161.52 72.16) (end 160.02 73.66) (width 1) (layer B.Cu) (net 12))
 (segment (start 160.02 73.66) (end 160.02 77.47) (width 1) (layer B.Cu) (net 12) (status 20))
 (segment (start 160.02 67.1575) (end 160.02 70.485) (width 0.8) (layer B.Cu) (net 11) (status 10))
 (segment (start 160.02 70.485) (end 157.48 73.025) (width 1) (layer B.Cu) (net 11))
 (segment (start 157.48 73.025) (end 157.48 77.47) (width 1) (layer B.Cu) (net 11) (status 20))
 (segment (start 155.52 49.6825) (end 155.52 37.41) (width 0.8) (layer B.Cu) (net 8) (status 10))
 (segment (start 154.94 36.83) (end 154.94 34.29) (width 1) (layer B.Cu) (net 8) (status 20))
 (segment (start 155.52 37.41) (end 154.94 36.83) (width 1) (layer B.Cu) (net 8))
 (segment (start 157.02 49.6825) (end 157.02 37.29) (width 0.8) (layer B.Cu) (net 7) (status 10))
 (segment (start 157.48 36.83) (end 157.48 34.29) (width 1) (layer B.Cu) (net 7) (status 20))
 (segment (start 157.02 37.29) (end 157.48 36.83) (width 1) (layer B.Cu) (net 7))
 (segment (start 150.495 82.55) (end 150.495 83.82) (width 1) (layer B.Cu) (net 16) (status 10))
 (segment (start 150.495 83.82) (end 151.765 85.09) (width 1) (layer B.Cu) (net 16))
 (segment (start 151.765 85.09) (end 154.94 85.09) (width 1) (layer B.Cu) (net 16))
 (segment (start 154.94 85.09) (end 158.75 88.9) (width 1) (layer B.Cu) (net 16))
 (segment (start 156.21 97.79) (end 158.75 97.79) (width 1) (layer B.Cu) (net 16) (status 10))
 (segment (start 158.75 88.9) (end 158.75 97.79) (width 1) (layer B.Cu) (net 16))
 (segment (start 158.75 97.79) (end 171.45 97.79) (width 1) (layer B.Cu) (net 16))
 (segment (start 171.45 92.71) (end 171.45 97.79) (width 1) (layer B.Cu) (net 16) (status 10))
 (segment (start 155.52 67.1575) (end 155.52 68.762) (width 0.8) (layer B.Cu) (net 9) (status 10))
 (segment (start 151.892 72.39) (end 150.495 72.39) (width 0.8) (layer B.Cu) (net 9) (status 20))
 (segment (start 155.52 68.762) (end 151.892 72.39) (width 0.8) (layer B.Cu) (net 9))
 (segment (start 163.83 87.63) (end 180.2892 87.63) (width 0.8) (layer B.Cu) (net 6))
 (segment (start 180.2892 87.63) (end 180.4924 87.4268) (width 0.8) (layer B.Cu) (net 6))
 (segment (start 180.4924 87.4268) (end 180.4924 38.608) (width 0.8) (layer B.Cu) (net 6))
 (segment (start 180.4924 38.608) (end 180.2892 38.4048) (width 0.8) (layer B.Cu) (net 6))
 (segment (start 180.2892 38.4048) (end 161.1884 38.4048) (width 0.8) (layer B.Cu) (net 6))
 (segment (start 161.1884 38.4048) (end 160.0708 39.5224) (width 0.8) (layer B.Cu) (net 6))
 (segment (start 159.9184 39.5224) (end 159.9184 41.7576) (width 0.8) (layer B.Cu) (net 6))
 (segment (start 160.0708 41.7576) (end 161.036 42.7228) (width 0.8) (layer B.Cu) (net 6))
 (segment (start 161.036 42.7228) (end 161.29 42.7228) (width 0.8) (layer B.Cu) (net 6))
 (segment (start 161.29 42.7228) (end 162.306 43.7388) (width 0.8) (layer B.Cu) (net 6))
 (segment (start 162.306 43.7388) (end 162.306 45.5676) (width 0.8) (layer B.Cu) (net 6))
 (segment (start 161.52 46.3536) (end 161.52 49.6825) (width 0.8) (layer B.Cu) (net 6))
 (segment (start 162.306 45.5676) (end 161.52 46.3536) (width 0.8) (layer B.Cu) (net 6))
 (segment (start 160.02 49.6825) (end 160.02 44.45) (width 0.8) (layer B.Cu) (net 3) (status 30))
 (segment (start 158.88863 44.45) (end 160.02 44.45) (width 0.8) (layer B.Cu) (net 3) (status 20))
 (segment (start 158.369 43.93037) (end 158.88863 44.45) (width 0.8) (layer B.Cu) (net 3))
 (segment (start 158.369 39.116) (end 158.369 43.93037) (width 0.8) (layer B.Cu) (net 3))
 (segment (start 158.75 38.735) (end 158.369 39.116) (width 0.8) (layer B.Cu) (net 3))
 (segment (start 182.245 36.83) (end 160.02 36.83) (width 0.8) (layer B.Cu) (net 3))
 (segment (start 182.372 36.957) (end 182.245 36.83) (width 1) (layer B.Cu) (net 3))
 (segment (start 182.118 101.6) (end 182.372 101.346) (width 1) (layer B.Cu) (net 3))
 (segment (start 182.372 101.346) (end 182.372 36.957) (width 1) (layer B.Cu) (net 3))
 (segment (start 147.32 95.885) (end 147.32 101.6) (width 1) (layer B.Cu) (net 3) (status 10))
 (segment (start 147.32 101.6) (end 182.118 101.6) (width 1) (layer B.Cu) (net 3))
 (segment (start 158.75 38.1) (end 160.02 36.83) (width 1) (layer B.Cu) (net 3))
 (segment (start 158.75 38.735) (end 158.75 38.1) (width 1) (layer B.Cu) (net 3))
 (segment (start 157.02 67.1575) (end 157.02 70.564) (width 0.8) (layer B.Cu) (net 10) (status 10))
 (segment (start 157.02 70.564) (end 156.512 70.564) (width 1) (layer B.Cu) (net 10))
 (segment (start 154.94 72.136) (end 154.94 73.95099) (width 1) (layer B.Cu) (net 10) (status 20))
 (segment (start 156.512 70.564) (end 154.94 72.136) (width 1) (layer B.Cu) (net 10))
 (segment (start 164.52 67.1575) (end 164.52 67.89) (width 0.8) (layer B.Cu) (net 14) (status 10))
 (segment (start 164.52 67.89) (end 164.52 68.144) (width 0.8) (layer B.Cu) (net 14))
 (segment (start 164.52 68.144) (end 164.084 68.58) (width 0.8) (layer B.Cu) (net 14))
 (segment (start 164.084 68.58) (end 163.83 68.58) (width 0.8) (layer B.Cu) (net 14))
 (segment (start 163.83 68.58) (end 163.322 69.088) (width 0.8) (layer B.Cu) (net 14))
 (segment (start 163.322 69.088) (end 163.322 71.882) (width 0.8) (layer B.Cu) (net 14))
 (segment (start 163.322 71.882) (end 163.576 72.136) (width 0.8) (layer B.Cu) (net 14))
 (via (at 163.576 72.136) (size 1.6) (drill 0.8) (layers F.Cu B.Cu) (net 14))
 (via (at 163.576 72.136) (size 0.8) (drill 0.4) (layers F.Cu B.Cu) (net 14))
 (segment (start 163.576 72.136) (end 168.148 72.136) (width 0.8) (layer F.Cu) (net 14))
 (via (at 168.148 72.136) (size 1.6) (drill 0.8) (layers F.Cu B.Cu) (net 14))
 (segment (start 177.486999 74.422) (end 177.546 74.422) (width 1) (layer B.Cu) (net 14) (status 30))
 (segment (start 177.546 72.136) (end 177.546 73.95099) (width 1) (layer B.Cu) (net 14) (status 20))
 (segment (start 177.546 72.136) (end 168.148 72.136) (width 1) (layer B.Cu) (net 14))
 (segment (start 153.67 82.55) (end 153.67 80.9244) (width 1) (layer B.Cu) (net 17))
 (segment (start 153.67 80.9244) (end 151.4856 78.74) (width 1) (layer B.Cu) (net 17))
 (segment (start 150.4696 77.724) (end 143.97607 77.724) (width 1) (layer B.Cu) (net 17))
 (segment (start 151.4856 78.74) (end 150.4696 77.724) (width 1) (layer B.Cu) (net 17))
 (segment (start 143.97607 77.724) (end 143.834649 77.724) (width 0.8) (layer B.Cu) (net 17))
 (segment (start 143.330639 77.21999) (end 142.875 77.21999) (width 0.8) (layer B.Cu) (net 17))
 (segment (start 143.834649 77.724) (end 143.330639 77.21999) (width 0.8) (layer B.Cu) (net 17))
 (segment (start 134.025 53.15) (end 134.025 49.871) (width 1) (layer B.Cu) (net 22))
 (segment (start 135.3312 48.5648) (end 138.4808 48.5648) (width 1) (layer B.Cu) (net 22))
 (segment (start 134.025 49.871) (end 135.3312 48.5648) (width 1) (layer B.Cu) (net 22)))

